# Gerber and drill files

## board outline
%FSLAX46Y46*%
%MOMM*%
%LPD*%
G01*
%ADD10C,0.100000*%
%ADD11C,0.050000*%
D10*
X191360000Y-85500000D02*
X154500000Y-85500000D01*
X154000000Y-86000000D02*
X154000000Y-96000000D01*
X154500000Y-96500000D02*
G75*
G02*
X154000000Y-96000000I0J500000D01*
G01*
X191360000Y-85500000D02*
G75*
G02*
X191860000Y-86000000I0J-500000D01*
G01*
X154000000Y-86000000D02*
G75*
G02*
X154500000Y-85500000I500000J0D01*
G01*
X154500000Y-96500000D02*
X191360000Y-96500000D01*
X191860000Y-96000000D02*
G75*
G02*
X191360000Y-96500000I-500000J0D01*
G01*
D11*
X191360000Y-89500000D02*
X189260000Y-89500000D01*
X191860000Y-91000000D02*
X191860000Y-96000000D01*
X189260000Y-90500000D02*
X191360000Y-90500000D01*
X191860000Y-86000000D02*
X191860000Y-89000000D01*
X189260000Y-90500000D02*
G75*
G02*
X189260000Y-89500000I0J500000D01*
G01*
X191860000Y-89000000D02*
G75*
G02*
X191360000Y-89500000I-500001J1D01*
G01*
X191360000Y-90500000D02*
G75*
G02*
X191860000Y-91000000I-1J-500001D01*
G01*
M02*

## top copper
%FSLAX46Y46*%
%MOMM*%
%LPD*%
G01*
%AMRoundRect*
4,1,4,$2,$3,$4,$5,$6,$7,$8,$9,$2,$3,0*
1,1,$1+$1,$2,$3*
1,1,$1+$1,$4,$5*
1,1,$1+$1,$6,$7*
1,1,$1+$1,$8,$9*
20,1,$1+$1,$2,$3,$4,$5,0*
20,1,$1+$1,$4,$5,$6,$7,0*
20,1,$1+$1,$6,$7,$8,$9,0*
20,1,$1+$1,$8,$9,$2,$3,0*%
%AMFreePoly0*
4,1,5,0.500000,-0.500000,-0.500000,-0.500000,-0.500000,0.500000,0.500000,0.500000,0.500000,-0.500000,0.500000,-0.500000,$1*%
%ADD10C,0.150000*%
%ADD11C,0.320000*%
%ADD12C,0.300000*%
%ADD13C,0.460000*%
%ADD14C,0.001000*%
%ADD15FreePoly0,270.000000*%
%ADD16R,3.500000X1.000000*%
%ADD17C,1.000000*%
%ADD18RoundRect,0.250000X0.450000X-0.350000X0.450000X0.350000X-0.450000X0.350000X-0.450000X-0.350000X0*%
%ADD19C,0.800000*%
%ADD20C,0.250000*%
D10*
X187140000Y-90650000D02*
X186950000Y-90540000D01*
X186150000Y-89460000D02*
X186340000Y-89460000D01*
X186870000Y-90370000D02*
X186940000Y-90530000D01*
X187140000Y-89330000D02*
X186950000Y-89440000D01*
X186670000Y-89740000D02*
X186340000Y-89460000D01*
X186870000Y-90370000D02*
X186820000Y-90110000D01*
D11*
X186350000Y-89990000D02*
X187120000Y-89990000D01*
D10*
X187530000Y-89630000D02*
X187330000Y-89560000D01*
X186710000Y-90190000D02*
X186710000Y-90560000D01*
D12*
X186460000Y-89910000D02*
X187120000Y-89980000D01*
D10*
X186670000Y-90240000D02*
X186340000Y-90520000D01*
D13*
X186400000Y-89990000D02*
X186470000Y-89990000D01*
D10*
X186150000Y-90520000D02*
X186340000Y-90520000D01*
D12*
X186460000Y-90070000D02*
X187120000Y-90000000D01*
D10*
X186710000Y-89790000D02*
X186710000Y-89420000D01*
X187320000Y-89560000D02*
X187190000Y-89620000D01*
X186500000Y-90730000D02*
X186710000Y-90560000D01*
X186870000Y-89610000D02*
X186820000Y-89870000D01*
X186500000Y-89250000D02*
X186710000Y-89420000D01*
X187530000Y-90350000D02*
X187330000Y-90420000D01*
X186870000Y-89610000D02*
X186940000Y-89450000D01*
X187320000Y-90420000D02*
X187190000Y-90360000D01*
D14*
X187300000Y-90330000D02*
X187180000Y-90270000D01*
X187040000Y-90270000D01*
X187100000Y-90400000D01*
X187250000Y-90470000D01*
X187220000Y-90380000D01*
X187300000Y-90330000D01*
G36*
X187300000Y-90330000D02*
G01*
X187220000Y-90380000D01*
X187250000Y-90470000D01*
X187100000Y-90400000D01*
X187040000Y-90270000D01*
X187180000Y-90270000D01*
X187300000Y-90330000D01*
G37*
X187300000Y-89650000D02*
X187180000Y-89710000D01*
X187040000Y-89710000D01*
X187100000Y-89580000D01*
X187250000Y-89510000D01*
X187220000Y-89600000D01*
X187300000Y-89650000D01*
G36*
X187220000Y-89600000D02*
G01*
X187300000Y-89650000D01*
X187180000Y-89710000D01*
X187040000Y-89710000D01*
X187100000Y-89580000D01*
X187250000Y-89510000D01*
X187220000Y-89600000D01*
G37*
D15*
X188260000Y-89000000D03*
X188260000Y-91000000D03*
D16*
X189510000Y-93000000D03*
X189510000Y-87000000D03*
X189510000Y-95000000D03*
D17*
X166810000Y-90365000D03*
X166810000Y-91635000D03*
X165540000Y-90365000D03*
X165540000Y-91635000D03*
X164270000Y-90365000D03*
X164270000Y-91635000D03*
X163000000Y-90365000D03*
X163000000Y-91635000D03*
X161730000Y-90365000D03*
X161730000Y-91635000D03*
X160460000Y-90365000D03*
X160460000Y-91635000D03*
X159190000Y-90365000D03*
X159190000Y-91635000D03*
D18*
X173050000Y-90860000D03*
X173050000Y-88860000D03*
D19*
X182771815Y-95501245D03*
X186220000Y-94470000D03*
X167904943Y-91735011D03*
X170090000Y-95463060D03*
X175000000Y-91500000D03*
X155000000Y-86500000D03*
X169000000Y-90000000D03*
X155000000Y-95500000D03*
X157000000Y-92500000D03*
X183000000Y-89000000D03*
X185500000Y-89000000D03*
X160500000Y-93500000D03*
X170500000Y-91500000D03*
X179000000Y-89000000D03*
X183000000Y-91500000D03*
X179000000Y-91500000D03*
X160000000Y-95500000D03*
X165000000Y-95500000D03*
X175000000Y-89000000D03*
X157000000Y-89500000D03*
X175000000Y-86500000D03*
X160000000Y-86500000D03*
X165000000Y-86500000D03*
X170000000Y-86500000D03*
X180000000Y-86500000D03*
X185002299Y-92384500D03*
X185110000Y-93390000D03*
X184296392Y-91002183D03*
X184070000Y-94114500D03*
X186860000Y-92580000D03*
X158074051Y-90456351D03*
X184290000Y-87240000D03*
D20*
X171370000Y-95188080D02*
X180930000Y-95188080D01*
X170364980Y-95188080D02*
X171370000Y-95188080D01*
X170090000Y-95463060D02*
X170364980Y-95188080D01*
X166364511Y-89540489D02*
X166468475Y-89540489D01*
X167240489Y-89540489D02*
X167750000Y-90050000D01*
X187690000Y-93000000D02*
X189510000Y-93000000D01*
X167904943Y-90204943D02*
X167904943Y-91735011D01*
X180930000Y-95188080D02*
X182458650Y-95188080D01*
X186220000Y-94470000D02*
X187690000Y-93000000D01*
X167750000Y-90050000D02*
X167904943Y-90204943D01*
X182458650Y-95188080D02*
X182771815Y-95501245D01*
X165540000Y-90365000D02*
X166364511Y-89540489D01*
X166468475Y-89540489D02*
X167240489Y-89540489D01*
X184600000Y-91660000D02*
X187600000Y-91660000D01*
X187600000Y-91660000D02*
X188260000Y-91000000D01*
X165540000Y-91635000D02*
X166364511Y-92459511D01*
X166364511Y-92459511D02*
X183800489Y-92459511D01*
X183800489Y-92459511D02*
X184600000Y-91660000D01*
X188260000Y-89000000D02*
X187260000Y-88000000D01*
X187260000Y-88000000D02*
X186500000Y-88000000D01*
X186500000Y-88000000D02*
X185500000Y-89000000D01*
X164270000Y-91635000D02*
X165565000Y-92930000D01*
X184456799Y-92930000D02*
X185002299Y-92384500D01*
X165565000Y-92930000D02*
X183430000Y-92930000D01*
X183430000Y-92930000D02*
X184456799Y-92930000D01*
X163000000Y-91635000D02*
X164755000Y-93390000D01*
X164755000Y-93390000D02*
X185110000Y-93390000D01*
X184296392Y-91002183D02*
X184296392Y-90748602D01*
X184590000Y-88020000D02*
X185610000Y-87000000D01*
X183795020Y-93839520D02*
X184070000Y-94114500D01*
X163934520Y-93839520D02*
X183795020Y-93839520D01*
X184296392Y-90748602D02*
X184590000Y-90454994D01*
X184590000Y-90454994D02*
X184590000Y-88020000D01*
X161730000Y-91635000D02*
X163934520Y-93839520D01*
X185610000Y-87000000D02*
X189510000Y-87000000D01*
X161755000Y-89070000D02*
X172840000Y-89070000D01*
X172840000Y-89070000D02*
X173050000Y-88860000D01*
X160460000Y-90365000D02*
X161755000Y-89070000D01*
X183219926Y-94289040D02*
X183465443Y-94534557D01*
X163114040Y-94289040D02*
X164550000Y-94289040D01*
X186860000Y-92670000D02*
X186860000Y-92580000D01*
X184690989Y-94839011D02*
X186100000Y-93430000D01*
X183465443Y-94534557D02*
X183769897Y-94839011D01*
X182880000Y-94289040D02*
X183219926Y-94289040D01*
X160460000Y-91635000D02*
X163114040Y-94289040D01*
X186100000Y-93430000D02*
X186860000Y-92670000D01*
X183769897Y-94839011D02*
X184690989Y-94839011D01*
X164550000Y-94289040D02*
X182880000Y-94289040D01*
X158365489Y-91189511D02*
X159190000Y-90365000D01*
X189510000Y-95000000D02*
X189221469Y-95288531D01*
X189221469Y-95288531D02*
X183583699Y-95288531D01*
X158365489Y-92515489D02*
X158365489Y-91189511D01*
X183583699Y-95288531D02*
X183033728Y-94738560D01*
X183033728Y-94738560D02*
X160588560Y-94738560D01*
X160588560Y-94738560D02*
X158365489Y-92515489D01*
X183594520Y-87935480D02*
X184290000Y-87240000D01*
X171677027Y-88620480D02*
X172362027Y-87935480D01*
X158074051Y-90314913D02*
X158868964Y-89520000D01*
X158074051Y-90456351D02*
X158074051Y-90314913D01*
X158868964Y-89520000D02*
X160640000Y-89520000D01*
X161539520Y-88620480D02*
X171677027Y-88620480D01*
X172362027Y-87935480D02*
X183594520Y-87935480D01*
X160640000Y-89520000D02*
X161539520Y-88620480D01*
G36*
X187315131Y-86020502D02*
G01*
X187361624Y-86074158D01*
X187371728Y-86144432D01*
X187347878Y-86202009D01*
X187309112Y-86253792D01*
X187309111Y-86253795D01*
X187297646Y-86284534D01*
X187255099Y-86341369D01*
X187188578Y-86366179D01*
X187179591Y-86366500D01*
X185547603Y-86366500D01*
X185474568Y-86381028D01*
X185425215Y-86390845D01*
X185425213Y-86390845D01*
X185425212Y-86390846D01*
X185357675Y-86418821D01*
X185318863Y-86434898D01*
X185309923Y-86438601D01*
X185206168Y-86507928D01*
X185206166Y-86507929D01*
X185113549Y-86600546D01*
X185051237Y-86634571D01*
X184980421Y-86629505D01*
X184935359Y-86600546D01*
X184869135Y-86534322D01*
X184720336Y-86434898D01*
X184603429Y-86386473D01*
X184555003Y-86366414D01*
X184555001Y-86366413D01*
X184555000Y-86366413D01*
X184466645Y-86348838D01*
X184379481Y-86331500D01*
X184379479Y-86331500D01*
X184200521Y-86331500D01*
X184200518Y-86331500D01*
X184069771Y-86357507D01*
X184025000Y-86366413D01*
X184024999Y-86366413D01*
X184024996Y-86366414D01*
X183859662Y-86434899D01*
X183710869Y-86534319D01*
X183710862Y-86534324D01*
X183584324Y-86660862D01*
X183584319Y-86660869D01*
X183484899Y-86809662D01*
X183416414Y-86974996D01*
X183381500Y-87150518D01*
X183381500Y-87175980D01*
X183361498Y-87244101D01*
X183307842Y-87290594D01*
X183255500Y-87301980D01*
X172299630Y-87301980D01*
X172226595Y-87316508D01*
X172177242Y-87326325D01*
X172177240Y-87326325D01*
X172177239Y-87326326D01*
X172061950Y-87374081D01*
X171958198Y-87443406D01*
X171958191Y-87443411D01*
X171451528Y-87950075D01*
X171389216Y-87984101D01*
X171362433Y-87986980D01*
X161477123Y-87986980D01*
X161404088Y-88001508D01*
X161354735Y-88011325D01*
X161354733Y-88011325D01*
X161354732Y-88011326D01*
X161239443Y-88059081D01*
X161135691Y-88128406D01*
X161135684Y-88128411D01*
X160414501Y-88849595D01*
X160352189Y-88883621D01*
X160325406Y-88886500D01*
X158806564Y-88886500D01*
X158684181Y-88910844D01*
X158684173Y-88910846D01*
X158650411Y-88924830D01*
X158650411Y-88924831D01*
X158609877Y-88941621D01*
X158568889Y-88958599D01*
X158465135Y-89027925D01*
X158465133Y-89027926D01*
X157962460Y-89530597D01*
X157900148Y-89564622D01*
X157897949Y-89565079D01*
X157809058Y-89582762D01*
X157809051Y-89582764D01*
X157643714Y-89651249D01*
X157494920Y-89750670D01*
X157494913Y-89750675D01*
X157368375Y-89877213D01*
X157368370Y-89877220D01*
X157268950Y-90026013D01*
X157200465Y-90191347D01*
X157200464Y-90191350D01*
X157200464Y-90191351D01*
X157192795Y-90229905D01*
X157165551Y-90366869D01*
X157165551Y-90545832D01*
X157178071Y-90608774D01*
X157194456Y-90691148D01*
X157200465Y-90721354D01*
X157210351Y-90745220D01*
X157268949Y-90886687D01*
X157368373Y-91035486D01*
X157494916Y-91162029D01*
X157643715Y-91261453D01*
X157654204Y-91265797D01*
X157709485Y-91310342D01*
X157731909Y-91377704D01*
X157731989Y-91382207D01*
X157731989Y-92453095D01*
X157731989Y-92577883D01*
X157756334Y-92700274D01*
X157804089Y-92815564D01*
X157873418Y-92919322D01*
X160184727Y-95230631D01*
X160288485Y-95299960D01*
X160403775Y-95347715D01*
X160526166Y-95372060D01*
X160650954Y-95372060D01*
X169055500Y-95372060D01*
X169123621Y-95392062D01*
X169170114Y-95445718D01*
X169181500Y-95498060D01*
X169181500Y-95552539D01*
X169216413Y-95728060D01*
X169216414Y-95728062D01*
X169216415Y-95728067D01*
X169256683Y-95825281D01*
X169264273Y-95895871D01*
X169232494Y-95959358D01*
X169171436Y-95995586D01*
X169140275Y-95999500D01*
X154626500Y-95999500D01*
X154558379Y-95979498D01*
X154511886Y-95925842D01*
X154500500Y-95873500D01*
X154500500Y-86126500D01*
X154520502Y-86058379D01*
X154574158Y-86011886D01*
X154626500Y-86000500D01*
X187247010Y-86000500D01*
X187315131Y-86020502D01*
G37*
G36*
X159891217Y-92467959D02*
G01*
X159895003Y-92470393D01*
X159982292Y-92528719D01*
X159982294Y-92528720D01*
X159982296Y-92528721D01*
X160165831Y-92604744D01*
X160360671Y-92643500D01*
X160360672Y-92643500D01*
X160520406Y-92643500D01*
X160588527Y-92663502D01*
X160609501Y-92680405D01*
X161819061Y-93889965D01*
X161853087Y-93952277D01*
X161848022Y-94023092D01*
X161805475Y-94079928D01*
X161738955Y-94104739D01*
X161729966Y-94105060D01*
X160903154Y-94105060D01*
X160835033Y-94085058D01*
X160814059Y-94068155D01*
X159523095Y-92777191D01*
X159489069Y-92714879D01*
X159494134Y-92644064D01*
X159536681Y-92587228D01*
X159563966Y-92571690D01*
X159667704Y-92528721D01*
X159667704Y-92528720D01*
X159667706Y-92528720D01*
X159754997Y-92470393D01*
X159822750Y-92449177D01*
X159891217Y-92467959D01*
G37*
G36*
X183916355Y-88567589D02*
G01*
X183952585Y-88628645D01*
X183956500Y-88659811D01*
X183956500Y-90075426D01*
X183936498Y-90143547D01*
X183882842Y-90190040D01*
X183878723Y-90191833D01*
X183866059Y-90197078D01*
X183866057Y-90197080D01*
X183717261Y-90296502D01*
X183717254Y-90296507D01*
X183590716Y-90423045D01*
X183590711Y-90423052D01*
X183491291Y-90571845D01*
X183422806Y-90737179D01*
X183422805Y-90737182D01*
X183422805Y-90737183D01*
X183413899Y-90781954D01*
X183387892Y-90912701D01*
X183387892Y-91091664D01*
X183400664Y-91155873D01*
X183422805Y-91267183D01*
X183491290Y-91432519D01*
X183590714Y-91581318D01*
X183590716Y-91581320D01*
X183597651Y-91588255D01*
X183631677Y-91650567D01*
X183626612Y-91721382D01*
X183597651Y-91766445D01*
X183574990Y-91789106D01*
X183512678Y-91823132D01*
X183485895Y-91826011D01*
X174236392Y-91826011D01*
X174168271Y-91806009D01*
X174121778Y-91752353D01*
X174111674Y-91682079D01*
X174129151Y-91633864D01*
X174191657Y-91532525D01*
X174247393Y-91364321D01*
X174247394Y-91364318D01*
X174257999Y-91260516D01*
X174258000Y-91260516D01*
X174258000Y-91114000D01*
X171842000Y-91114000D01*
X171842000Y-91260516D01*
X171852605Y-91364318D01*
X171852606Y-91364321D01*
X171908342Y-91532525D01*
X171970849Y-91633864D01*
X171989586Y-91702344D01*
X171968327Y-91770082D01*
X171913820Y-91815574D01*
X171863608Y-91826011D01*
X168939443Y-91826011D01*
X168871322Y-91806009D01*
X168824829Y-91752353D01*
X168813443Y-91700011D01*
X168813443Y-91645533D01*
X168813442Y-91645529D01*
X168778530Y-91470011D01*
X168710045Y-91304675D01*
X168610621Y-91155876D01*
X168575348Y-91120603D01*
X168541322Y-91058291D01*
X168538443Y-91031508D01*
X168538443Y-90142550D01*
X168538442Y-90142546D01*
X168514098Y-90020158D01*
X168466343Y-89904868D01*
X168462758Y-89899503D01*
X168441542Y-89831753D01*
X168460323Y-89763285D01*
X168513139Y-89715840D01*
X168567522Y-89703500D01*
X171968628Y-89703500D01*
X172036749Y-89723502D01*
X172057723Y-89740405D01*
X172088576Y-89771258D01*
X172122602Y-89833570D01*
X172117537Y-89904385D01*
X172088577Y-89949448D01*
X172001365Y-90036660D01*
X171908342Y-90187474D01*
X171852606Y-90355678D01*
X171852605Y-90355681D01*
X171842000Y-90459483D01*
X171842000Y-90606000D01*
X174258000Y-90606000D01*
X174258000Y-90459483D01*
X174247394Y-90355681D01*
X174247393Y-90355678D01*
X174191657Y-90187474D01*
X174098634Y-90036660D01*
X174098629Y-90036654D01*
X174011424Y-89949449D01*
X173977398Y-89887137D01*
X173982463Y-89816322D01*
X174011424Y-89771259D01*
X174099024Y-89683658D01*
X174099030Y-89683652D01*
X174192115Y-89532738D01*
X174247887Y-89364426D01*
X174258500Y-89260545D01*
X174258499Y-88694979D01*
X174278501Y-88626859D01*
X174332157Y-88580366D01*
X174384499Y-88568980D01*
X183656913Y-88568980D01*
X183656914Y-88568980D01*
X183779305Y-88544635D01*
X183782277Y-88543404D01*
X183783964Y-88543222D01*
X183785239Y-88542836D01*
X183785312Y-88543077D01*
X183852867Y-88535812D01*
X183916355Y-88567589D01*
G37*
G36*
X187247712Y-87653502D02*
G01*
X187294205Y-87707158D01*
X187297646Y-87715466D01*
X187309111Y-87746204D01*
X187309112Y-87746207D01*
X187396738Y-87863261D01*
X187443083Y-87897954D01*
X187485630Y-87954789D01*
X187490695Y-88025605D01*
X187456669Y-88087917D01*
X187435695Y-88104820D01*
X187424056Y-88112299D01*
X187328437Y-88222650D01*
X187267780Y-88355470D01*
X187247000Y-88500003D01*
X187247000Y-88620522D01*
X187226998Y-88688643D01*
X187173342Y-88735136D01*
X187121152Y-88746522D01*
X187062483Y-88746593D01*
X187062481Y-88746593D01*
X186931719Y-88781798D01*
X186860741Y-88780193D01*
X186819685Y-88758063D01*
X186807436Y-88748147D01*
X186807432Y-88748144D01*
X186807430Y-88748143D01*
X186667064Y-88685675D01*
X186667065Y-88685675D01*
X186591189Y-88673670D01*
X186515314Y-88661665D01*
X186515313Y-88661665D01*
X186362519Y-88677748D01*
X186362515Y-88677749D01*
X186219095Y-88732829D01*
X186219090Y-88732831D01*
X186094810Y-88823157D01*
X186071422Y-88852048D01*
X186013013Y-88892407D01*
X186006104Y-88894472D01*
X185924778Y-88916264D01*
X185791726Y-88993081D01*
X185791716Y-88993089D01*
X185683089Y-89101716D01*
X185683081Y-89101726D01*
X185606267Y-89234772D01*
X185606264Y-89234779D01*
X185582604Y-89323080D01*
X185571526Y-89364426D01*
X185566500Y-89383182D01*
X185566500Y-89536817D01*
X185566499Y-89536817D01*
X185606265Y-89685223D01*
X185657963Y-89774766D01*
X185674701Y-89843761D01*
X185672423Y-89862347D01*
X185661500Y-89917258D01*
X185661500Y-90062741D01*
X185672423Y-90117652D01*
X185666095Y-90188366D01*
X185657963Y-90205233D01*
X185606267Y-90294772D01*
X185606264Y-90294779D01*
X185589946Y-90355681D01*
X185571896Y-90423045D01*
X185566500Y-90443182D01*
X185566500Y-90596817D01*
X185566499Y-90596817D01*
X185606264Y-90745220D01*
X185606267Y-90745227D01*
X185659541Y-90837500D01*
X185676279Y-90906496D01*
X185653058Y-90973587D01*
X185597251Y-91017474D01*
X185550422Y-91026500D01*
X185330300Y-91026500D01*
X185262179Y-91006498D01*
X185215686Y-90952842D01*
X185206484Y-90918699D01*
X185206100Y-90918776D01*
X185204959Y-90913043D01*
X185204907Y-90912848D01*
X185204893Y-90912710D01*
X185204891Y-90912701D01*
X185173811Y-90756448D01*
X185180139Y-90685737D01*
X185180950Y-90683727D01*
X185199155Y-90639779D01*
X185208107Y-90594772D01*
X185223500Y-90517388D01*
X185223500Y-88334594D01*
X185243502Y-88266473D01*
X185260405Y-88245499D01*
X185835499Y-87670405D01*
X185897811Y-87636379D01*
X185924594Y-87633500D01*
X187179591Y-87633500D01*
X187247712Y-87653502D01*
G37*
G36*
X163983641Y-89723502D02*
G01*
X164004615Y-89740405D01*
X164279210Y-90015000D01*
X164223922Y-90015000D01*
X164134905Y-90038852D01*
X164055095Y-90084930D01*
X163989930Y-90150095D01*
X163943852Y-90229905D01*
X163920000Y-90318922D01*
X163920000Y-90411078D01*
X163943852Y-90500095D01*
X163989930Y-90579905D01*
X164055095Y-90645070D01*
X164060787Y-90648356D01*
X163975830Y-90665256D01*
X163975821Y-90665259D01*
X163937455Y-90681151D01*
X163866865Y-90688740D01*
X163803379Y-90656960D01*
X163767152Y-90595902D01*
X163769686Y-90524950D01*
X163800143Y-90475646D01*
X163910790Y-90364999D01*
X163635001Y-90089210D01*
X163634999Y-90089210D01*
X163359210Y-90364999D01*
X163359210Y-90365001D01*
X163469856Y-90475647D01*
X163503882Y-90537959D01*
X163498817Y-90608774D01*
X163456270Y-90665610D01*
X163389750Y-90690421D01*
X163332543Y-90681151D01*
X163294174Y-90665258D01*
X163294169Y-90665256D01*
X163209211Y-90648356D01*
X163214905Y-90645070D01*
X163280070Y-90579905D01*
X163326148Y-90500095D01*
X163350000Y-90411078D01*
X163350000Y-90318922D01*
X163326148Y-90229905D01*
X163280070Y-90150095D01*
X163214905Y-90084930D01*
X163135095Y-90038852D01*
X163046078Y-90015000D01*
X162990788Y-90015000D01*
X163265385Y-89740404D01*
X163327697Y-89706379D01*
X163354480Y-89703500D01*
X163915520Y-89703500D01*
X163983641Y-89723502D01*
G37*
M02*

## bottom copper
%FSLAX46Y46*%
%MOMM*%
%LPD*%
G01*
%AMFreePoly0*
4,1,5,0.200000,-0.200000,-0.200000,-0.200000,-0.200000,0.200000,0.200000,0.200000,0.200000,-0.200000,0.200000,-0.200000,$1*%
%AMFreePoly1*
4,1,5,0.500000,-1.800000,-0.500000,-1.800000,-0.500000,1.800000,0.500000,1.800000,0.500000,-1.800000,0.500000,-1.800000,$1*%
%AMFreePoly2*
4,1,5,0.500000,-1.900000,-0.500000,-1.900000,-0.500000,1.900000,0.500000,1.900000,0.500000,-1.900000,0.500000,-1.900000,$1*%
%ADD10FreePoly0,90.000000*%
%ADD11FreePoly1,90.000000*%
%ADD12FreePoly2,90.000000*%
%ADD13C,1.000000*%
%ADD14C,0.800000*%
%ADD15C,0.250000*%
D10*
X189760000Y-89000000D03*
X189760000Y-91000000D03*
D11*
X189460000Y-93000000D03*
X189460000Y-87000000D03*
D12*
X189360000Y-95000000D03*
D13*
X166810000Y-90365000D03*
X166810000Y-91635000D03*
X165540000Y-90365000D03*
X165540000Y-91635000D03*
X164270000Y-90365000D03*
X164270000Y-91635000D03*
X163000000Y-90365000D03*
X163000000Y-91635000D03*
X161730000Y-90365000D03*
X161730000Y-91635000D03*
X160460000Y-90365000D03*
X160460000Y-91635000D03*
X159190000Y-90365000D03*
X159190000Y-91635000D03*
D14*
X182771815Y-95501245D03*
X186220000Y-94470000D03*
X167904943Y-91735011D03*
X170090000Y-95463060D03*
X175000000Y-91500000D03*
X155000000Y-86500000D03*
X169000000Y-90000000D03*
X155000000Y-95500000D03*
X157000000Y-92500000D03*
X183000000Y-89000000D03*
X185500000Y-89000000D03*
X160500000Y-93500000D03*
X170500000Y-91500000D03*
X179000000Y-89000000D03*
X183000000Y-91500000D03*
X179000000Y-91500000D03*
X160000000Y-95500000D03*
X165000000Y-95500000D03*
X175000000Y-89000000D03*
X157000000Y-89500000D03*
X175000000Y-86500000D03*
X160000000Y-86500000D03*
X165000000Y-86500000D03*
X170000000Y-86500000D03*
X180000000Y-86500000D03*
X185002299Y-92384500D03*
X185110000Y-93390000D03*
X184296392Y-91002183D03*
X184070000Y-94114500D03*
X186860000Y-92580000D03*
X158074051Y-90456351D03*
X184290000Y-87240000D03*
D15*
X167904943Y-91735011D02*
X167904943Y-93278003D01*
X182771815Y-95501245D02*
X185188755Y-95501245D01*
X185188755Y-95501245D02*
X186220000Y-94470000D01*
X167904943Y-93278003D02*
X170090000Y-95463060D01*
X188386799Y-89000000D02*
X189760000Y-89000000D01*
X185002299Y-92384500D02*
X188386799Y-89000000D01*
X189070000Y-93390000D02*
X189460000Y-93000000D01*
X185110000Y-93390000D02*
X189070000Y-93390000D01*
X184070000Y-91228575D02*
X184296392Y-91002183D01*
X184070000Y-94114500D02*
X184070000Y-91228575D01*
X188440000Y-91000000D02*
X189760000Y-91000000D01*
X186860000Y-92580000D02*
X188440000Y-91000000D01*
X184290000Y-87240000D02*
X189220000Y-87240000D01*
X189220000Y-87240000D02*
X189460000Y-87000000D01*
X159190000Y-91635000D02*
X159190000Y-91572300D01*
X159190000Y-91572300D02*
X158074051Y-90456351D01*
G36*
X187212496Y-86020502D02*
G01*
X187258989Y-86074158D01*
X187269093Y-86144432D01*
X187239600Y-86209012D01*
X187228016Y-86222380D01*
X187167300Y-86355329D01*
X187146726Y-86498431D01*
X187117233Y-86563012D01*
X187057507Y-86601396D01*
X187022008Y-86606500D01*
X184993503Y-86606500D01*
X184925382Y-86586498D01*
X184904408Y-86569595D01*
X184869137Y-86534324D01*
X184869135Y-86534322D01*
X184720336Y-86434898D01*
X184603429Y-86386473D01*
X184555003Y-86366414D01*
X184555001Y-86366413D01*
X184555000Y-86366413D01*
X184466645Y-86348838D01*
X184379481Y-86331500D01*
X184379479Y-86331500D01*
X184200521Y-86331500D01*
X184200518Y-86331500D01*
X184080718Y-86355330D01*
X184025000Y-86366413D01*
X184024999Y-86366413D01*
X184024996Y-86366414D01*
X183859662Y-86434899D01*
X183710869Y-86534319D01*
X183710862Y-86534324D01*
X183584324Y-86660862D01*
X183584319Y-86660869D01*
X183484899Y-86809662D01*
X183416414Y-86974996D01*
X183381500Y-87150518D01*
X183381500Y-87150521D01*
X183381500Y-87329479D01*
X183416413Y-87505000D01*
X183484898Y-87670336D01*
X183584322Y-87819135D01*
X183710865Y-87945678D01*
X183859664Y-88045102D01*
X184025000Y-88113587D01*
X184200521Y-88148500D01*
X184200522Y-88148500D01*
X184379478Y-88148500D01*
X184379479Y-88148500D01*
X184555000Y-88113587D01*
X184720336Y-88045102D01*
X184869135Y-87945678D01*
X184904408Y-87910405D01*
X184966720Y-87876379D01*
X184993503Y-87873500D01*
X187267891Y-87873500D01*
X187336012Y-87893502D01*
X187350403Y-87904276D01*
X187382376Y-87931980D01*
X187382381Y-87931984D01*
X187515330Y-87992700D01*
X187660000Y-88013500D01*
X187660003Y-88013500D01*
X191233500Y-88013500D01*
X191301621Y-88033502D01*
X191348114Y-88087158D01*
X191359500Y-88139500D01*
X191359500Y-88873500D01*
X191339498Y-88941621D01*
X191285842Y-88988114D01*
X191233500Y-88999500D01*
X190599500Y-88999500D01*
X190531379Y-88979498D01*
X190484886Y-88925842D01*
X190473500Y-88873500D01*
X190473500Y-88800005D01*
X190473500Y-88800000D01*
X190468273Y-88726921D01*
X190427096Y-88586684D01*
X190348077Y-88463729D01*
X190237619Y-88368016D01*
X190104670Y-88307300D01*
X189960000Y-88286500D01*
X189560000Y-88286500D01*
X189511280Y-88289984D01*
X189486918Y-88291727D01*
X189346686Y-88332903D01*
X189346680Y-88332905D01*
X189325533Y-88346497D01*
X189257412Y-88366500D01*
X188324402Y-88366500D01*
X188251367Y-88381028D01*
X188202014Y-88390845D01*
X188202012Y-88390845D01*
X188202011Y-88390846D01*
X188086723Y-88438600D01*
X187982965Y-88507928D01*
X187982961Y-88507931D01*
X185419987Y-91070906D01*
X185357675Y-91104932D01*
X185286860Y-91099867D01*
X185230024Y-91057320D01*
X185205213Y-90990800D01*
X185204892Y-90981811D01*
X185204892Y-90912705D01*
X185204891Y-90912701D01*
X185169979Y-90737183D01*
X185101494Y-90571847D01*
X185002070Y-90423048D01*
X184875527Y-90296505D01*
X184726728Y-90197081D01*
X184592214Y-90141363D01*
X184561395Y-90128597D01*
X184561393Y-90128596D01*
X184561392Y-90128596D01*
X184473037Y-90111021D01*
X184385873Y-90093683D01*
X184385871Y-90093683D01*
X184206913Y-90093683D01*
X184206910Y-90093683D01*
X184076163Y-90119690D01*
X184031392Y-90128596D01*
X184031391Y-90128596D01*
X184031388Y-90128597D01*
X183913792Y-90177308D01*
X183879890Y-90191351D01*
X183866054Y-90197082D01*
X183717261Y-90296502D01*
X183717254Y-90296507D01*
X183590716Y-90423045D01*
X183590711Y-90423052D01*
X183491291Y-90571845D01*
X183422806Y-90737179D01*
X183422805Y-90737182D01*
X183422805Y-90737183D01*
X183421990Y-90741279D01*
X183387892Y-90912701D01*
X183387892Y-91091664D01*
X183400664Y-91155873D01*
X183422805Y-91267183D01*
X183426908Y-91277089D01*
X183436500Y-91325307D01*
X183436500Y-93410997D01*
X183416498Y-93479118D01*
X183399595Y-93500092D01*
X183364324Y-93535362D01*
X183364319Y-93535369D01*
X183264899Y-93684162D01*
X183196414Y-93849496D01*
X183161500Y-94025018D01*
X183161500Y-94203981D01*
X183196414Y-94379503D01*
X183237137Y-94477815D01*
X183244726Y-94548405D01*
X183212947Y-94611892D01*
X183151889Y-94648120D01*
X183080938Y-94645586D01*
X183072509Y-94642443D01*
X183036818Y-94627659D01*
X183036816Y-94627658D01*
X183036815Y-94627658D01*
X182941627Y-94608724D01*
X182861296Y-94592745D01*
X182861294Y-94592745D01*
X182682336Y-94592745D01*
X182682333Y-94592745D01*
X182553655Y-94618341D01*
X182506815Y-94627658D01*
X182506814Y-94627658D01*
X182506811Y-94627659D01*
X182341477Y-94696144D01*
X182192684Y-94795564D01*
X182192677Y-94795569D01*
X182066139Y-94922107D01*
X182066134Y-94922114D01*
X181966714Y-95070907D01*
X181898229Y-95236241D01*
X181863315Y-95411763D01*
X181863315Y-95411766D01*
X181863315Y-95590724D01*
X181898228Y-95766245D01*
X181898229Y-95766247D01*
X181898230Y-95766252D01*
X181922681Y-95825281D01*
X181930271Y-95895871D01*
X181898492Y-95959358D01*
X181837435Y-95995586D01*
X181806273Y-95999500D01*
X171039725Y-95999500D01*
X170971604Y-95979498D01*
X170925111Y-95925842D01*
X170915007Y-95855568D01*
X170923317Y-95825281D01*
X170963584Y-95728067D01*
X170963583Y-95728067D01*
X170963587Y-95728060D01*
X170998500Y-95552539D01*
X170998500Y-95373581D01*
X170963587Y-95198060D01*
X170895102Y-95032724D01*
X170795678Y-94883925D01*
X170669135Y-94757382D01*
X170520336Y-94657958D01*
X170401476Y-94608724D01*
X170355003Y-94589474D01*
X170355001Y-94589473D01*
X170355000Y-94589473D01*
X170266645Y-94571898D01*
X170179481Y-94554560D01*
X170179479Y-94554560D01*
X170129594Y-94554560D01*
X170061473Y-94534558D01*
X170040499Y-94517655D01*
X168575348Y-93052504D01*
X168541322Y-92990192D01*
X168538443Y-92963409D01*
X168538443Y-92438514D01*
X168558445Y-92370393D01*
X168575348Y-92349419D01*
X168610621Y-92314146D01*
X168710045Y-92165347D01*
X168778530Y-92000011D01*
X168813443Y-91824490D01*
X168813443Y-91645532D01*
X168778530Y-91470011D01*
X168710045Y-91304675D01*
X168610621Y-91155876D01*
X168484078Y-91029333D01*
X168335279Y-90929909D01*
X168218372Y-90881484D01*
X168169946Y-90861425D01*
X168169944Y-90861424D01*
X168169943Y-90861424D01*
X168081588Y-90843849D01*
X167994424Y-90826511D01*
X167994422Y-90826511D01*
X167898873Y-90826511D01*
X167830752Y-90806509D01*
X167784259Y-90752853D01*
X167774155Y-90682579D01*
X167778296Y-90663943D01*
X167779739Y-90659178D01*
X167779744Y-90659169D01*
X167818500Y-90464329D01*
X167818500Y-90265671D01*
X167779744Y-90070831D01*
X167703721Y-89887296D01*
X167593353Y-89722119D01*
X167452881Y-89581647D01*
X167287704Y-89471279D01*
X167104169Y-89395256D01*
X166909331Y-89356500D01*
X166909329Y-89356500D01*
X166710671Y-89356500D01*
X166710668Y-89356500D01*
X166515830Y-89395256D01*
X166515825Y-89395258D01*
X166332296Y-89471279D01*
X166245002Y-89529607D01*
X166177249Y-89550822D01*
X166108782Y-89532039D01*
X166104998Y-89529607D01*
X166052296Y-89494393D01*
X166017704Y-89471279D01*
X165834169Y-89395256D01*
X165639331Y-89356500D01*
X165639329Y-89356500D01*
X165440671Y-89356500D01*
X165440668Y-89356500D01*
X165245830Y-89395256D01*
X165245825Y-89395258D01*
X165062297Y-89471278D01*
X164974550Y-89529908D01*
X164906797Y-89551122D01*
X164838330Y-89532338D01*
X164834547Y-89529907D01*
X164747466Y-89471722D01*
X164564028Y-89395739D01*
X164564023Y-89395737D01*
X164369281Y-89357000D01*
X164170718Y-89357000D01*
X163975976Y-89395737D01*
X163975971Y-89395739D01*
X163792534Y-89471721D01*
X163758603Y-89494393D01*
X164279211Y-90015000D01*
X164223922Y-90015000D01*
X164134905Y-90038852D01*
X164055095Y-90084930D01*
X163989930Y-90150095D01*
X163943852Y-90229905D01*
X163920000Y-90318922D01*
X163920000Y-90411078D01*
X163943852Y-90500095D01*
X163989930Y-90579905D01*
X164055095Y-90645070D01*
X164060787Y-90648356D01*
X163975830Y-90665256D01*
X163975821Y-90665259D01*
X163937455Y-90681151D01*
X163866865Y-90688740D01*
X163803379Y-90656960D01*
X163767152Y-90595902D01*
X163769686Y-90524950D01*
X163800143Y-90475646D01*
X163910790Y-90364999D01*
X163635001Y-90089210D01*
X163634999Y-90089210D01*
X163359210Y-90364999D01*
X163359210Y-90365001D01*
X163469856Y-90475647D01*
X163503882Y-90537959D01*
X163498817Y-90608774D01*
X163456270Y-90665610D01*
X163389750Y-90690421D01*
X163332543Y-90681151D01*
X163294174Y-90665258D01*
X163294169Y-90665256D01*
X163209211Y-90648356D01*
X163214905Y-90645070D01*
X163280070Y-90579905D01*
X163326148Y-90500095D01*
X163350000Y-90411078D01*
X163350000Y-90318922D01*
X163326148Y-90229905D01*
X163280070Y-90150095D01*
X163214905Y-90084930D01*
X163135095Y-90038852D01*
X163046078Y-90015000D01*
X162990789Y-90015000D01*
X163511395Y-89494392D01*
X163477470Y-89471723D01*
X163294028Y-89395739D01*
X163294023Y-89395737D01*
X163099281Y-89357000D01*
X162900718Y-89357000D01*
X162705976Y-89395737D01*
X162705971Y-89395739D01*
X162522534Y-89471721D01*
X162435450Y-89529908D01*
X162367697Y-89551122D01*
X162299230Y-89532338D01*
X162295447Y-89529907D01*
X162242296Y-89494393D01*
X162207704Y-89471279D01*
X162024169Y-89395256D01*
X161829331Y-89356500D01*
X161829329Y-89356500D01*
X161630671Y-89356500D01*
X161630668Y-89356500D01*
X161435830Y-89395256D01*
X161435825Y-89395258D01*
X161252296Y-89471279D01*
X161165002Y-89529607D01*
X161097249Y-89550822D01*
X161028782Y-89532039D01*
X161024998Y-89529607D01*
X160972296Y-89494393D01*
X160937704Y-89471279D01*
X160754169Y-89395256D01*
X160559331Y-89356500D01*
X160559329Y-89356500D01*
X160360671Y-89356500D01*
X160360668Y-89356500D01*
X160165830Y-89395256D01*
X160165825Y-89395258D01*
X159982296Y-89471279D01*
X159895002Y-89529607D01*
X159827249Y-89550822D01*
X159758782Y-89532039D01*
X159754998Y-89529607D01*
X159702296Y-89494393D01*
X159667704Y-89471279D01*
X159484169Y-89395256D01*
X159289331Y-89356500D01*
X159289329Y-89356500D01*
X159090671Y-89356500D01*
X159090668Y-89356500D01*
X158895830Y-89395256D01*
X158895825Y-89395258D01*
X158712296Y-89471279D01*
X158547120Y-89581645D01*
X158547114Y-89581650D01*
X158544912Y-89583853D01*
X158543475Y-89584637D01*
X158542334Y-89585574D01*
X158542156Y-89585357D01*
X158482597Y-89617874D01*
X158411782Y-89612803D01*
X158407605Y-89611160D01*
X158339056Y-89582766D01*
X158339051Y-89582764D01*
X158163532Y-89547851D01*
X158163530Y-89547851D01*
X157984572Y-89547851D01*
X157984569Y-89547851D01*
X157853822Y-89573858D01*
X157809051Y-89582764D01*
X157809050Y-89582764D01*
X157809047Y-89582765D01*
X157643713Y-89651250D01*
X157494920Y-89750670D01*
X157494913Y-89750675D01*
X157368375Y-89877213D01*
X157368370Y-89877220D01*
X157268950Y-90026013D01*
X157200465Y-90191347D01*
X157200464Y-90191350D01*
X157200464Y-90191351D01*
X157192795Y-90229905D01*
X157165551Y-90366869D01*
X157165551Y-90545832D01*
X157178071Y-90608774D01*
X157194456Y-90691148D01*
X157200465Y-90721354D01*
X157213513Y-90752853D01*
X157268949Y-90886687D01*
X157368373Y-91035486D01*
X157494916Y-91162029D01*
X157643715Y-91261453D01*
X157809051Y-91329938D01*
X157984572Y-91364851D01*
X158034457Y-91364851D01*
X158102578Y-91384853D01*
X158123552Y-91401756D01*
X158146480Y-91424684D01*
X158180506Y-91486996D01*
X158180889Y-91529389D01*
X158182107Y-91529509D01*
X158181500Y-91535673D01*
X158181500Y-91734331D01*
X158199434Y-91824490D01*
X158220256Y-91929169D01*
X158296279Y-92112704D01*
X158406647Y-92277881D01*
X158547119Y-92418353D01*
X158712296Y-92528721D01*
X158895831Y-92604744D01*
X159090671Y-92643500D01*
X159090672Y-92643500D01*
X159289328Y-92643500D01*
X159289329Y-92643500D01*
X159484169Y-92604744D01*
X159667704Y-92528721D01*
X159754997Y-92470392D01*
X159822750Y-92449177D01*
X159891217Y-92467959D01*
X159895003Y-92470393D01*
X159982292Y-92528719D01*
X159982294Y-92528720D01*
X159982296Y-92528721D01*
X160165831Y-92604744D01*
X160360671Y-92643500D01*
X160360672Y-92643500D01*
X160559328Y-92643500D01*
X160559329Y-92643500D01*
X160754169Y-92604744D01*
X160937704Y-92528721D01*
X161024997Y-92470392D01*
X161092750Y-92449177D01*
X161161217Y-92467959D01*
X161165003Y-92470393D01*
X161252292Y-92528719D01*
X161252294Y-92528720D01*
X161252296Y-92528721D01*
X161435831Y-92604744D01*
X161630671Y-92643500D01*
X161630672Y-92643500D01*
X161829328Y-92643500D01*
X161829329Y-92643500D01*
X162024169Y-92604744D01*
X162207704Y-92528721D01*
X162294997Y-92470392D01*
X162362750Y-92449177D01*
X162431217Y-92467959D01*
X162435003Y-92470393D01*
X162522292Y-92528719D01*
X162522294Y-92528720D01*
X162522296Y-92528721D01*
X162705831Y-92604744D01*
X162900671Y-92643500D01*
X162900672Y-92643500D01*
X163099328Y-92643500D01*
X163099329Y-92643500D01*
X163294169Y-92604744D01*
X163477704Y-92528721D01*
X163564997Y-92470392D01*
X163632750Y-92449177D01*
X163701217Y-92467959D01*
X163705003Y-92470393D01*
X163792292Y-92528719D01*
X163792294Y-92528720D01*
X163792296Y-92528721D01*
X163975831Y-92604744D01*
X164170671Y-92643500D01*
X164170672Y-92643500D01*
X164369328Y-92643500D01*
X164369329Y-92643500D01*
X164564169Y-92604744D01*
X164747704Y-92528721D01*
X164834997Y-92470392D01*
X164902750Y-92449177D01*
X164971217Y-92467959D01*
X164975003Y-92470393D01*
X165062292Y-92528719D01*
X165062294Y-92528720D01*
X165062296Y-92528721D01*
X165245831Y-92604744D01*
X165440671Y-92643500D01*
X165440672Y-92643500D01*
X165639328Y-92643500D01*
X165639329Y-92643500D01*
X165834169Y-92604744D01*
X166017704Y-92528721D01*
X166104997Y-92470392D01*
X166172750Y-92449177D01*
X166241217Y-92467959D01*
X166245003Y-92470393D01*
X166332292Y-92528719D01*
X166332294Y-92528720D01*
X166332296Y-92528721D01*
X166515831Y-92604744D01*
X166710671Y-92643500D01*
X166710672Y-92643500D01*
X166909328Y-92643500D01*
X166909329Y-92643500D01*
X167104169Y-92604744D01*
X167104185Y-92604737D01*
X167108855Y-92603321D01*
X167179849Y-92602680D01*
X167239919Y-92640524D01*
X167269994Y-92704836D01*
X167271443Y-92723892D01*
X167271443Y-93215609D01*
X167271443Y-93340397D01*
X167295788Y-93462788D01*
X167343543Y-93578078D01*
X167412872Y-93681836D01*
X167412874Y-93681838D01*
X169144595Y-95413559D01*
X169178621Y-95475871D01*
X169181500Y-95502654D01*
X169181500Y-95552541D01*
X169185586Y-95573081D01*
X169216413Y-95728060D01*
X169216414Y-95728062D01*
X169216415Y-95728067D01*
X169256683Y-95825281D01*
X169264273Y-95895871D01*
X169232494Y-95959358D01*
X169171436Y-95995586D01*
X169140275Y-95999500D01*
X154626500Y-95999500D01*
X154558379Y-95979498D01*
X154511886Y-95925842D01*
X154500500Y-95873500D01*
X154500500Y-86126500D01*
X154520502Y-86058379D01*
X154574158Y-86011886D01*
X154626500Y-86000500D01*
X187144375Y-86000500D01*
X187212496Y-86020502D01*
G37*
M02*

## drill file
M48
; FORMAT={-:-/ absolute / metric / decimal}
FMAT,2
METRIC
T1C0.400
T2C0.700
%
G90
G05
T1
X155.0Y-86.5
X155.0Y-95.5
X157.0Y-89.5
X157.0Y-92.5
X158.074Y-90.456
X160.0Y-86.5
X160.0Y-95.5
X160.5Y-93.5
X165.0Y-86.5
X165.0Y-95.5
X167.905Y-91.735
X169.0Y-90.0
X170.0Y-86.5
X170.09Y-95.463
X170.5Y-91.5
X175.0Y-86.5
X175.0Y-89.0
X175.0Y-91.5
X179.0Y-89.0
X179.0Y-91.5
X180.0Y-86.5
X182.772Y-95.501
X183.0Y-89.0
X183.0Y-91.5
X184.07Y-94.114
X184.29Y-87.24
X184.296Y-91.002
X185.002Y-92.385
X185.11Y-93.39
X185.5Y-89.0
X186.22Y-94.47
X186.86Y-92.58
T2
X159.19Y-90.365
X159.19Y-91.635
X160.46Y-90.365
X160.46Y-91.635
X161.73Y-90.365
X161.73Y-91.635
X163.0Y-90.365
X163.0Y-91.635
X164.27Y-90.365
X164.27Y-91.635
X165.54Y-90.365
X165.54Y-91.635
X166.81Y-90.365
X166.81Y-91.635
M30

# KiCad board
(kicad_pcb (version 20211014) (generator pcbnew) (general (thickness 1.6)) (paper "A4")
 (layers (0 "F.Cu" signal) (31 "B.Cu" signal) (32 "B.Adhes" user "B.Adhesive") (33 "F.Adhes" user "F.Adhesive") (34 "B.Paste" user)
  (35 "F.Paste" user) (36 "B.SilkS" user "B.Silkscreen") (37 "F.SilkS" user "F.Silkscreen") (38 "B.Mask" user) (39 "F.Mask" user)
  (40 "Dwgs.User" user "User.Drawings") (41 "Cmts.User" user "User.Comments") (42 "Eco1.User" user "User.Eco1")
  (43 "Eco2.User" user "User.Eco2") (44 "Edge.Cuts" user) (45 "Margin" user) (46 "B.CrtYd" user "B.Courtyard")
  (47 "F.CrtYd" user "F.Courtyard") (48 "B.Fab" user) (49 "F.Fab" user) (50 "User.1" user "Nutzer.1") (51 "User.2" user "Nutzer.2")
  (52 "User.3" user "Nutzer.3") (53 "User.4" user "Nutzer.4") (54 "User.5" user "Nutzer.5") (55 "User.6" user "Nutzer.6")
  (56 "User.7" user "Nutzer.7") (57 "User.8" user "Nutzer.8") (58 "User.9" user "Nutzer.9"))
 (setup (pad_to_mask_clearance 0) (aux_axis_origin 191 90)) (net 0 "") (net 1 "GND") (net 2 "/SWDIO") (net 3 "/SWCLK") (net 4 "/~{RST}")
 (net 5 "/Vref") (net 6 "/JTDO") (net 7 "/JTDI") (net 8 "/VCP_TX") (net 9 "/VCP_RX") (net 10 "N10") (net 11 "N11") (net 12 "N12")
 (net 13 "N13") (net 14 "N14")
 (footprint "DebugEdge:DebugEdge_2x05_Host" (layer "F.Cu") (at 191.86 91 -90)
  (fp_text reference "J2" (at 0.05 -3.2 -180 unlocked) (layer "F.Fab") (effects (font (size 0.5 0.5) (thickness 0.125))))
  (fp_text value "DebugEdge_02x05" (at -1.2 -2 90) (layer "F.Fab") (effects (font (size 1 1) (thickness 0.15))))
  (fp_line (start -0.35 4.72) (end -0.46 4.91) (layer "F.Cu") (width 0.15))
  (fp_line (start -1.54 5.71) (end -1.54 5.52) (layer "F.Cu") (width 0.15))
  (fp_line (start -0.63 4.99) (end -0.47 4.92) (layer "F.Cu") (width 0.15))
  (fp_line (start -1.67 4.72) (end -1.56 4.91) (layer "F.Cu") (width 0.15))
  (fp_line (start -1.26 5.19) (end -1.54 5.52) (layer "F.Cu") (width 0.15))
  (fp_line (start -0.63 4.99) (end -0.89 5.04) (layer "F.Cu") (width 0.15))
  (fp_line (start -1.01 5.51) (end -1.01 4.74) (layer "F.Cu") (width 0.32))
  (fp_line (start -1.37 4.33) (end -1.44 4.53) (layer "F.Cu") (width 0.15))
  (fp_line (start -0.81 5.15) (end -0.44 5.15) (layer "F.Cu") (width 0.15))
  (fp_line (start -1.09 5.4) (end -1.02 4.74) (layer "F.Cu") (width 0.3))
  (fp_line (start -0.76 5.19) (end -0.48 5.52) (layer "F.Cu") (width 0.15))
  (fp_line (start -1.01 5.46) (end -1.01 5.39) (layer "F.Cu") (width 0.46))
  (fp_line (start -0.48 5.71) (end -0.48 5.52) (layer "F.Cu") (width 0.15))
  (fp_line (start -0.93 5.4) (end -1 4.74) (layer "F.Cu") (width 0.3))
  (fp_line (start -1.21 5.15) (end -1.58 5.15) (layer "F.Cu") (width 0.15))
  (fp_line (start -1.44 4.54) (end -1.38 4.67) (layer "F.Cu") (width 0.15))
  (fp_line (start -0.27 5.36) (end -0.44 5.15) (layer "F.Cu") (width 0.15))
  (fp_line (start -1.39 4.99) (end -1.13 5.04) (layer "F.Cu") (width 0.15))
  (fp_line (start -1.75 5.36) (end -1.58 5.15) (layer "F.Cu") (width 0.15))
  (fp_line (start -0.65 4.33) (end -0.58 4.53) (layer "F.Cu") (width 0.15))
  (fp_line (start -1.39 4.99) (end -1.55 4.92) (layer "F.Cu") (width 0.15))
  (fp_line (start -0.58 4.54) (end -0.64 4.67) (layer "F.Cu") (width 0.15))
  (fp_poly
   (pts (xy -0.67 4.56) (xy -0.73 4.68) (xy -0.73 4.82) (xy -0.6 4.76) (xy -0.53 4.61) (xy -0.62 4.64)) (layer "F.Cu") (width 0.001)
   (fill solid))
  (fp_poly
   (pts (xy -1.35 4.56) (xy -1.29 4.68) (xy -1.29 4.82) (xy -1.42 4.76) (xy -1.49 4.61) (xy -1.4 4.64)) (layer "F.Cu") (width 0.001)
   (fill solid))
  (fp_line (start -1.5 0.5) (end -1.5 2.6) (layer "Edge.Cuts") (width 0.05))
  (fp_line (start 0 0) (end 5 0) (layer "Edge.Cuts") (width 0.05))
  (fp_line (start -0.5 2.6) (end -0.5 0.5) (layer "Edge.Cuts") (width 0.05))
  (fp_line (start -5 0) (end -2 0) (layer "Edge.Cuts") (width 0.05))
  (fp_arc (start -0.5 2.6) (mid -1 3.1) (end -1.5 2.6) (layer "Edge.Cuts") (width 0.05))
  (fp_arc (start -2 0) (mid -1.646447 0.146447) (end -1.5 0.5) (layer "Edge.Cuts") (width 0.05))
  (fp_arc (start -0.5 0.5) (mid -0.353553 0.146447) (end 0 0) (layer "Edge.Cuts") (width 0.05))
  (pad "1" smd custom locked (at -2 3.6 270) (size 1 1) (layers "F.Cu" "F.Mask") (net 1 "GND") (zone_connect 0)
   (options (clearance outline) (anchor rect)) (primitives))
  (pad "2" smd custom locked (at 0 3.6 270) (size 1 1) (layers "F.Cu" "F.Mask") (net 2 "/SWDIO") (zone_connect 0)
   (options (clearance outline) (anchor rect)) (primitives))
  (pad "3" smd custom locked (at -2 2.1 90) (size 0.4 0.4) (layers "B.Cu" "B.Mask") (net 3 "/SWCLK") (zone_connect 0)
   (options (clearance outline) (anchor rect)) (primitives))
  (pad "4" smd custom locked (at 0 2.1 90) (size 0.4 0.4) (layers "B.Cu" "B.Mask") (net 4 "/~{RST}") (zone_connect 0)
   (options (clearance outline) (anchor rect)) (primitives))
  (pad "5" smd rect locked (at 2 2.35 270) (size 1 3.5) (layers "F.Cu" "F.Mask") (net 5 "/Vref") (zone_connect 0))
  (pad "6" smd custom locked (at 2 2.4 90) (size 1 3.6) (layers "B.Cu" "B.Mask") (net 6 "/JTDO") (zone_connect 0)
   (options (clearance outline) (anchor rect)) (primitives))
  (pad "7" smd rect locked (at -4 2.35 270) (size 1 3.5) (layers "F.Cu" "F.Mask") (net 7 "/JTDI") (zone_connect 0))
  (pad "8" smd custom locked (at -4 2.4 90) (size 1 3.6) (layers "B.Cu" "B.Mask") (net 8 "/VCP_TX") (zone_connect 0)
   (options (clearance outline) (anchor rect)) (primitives))
  (pad "9" smd rect locked (at 4 2.35 270) (size 1 3.5) (layers "F.Cu" "F.Mask") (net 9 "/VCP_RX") (zone_connect 0))
  (pad "10" smd custom locked (at 4 2.5 90) (size 1 3.8) (layers "B.Cu" "B.Mask") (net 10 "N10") (zone_connect 0)
   (options (clearance outline) (anchor rect)) (primitives)))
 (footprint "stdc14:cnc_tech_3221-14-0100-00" (layer "F.Cu") (at 163 91)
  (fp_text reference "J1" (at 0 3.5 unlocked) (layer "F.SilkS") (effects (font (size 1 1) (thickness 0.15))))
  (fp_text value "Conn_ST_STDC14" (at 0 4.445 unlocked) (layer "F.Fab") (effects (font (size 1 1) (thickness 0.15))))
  (pad "1" thru_hole circle (at 3.81 -0.635) (size 1 1) (drill 0.7) (layers *.Cu *.Mask) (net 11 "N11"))
  (pad "2" thru_hole circle (at 3.81 0.635) (size 1 1) (drill 0.7) (layers *.Cu *.Mask) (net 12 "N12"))
  (pad "3" thru_hole circle (at 2.54 -0.635) (size 1 1) (drill 0.7) (layers *.Cu *.Mask) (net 5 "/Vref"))
  (pad "4" thru_hole circle (at 2.54 0.635) (size 1 1) (drill 0.7) (layers *.Cu *.Mask) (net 2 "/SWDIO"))
  (pad "5" thru_hole circle (at 1.27 -0.635) (size 1 1) (drill 0.7) (layers *.Cu *.Mask) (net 1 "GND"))
  (pad "6" thru_hole circle (at 1.27 0.635) (size 1 1) (drill 0.7) (layers *.Cu *.Mask) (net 3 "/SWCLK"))
  (pad "7" thru_hole circle (at 0 -0.635) (size 1 1) (drill 0.7) (layers *.Cu *.Mask) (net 1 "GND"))
  (pad "8" thru_hole circle (at 0 0.635) (size 1 1) (drill 0.7) (layers *.Cu *.Mask) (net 6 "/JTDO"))
  (pad "9" thru_hole circle (at -1.27 -0.635) (size 1 1) (drill 0.7) (layers *.Cu *.Mask) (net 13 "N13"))
  (pad "10" thru_hole circle (at -1.27 0.635) (size 1 1) (drill 0.7) (layers *.Cu *.Mask) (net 7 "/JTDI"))
  (pad "11" thru_hole circle (at -2.54 -0.635) (size 1 1) (drill 0.7) (layers *.Cu *.Mask) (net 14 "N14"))
  (pad "12" thru_hole circle (at -2.54 0.635) (size 1 1) (drill 0.7) (layers *.Cu *.Mask) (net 4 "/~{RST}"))
  (pad "13" thru_hole circle (at -3.81 -0.635) (size 1 1) (drill 0.7) (layers *.Cu *.Mask) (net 9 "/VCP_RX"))
  (pad "14" thru_hole circle (at -3.81 0.635) (size 1 1) (drill 0.7) (layers *.Cu *.Mask) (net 8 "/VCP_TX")))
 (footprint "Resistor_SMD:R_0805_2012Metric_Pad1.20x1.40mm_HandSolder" (layer "F.Cu") (at 173.05 89.86 90)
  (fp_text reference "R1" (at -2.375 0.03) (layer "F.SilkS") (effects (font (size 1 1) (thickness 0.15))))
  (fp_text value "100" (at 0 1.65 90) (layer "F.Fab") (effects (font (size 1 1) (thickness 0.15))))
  (pad "1" smd roundrect (at -1 0 90) (size 1.2 1.4) (layers "F.Cu" "F.Paste" "F.Mask") (roundrect_rratio 0.208333) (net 1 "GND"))
  (pad "2" smd roundrect (at 1 0 90) (size 1.2 1.4) (layers "F.Cu" "F.Paste" "F.Mask") (roundrect_rratio 0.208333) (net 14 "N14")))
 (gr_line (start 191.36 85.5) (end 154.5 85.5) (layer "Edge.Cuts") (width 0.1))
 (gr_line (start 154 86) (end 154 96) (layer "Edge.Cuts") (width 0.1))
 (gr_arc (start 154.5 96.5) (mid 154.146447 96.353553) (end 154 96) (layer "Edge.Cuts") (width 0.1))
 (gr_arc (start 191.36 85.5) (mid 191.713553 85.646447) (end 191.86 86) (layer "Edge.Cuts") (width 0.1))
 (gr_arc (start 154 86) (mid 154.146447 85.646447) (end 154.5 85.5) (layer "Edge.Cuts") (width 0.1))
 (gr_line (start 154.5 96.5) (end 191.36 96.5) (layer "Edge.Cuts") (width 0.1))
 (gr_arc (start 191.86 96) (mid 191.713553 96.353553) (end 191.36 96.5) (layer "Edge.Cuts") (width 0.1))
 (segment (start 171.37 95.18808) (end 180.93 95.18808) (width 0.25) (layer "F.Cu") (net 5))
 (segment (start 170.36498 95.18808) (end 171.37 95.18808) (width 0.25) (layer "F.Cu") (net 5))
 (segment (start 170.09 95.46306) (end 170.36498 95.18808) (width 0.25) (layer "F.Cu") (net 5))
 (segment (start 166.364511 89.540489) (end 166.468475 89.540489) (width 0.25) (layer "F.Cu") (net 5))
 (segment (start 167.240489 89.540489) (end 167.75 90.05) (width 0.25) (layer "F.Cu") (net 5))
 (segment (start 187.69 93) (end 189.51 93) (width 0.25) (layer "F.Cu") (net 5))
 (segment (start 167.904943 90.204943) (end 167.904943 91.735011) (width 0.25) (layer "F.Cu") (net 5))
 (segment (start 180.93 95.18808) (end 182.45865 95.18808) (width 0.25) (layer "F.Cu") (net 5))
 (segment (start 186.22 94.47) (end 187.69 93) (width 0.25) (layer "F.Cu") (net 5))
 (segment (start 167.75 90.05) (end 167.904943 90.204943) (width 0.25) (layer "F.Cu") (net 5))
 (segment (start 182.45865 95.18808) (end 182.771815 95.501245) (width 0.25) (layer "F.Cu") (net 5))
 (segment (start 165.54 90.365) (end 166.364511 89.540489) (width 0.25) (layer "F.Cu") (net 5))
 (segment (start 166.468475 89.540489) (end 167.240489 89.540489) (width 0.25) (layer "F.Cu") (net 5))
 (via (at 182.771815 95.501245) (size 0.8) (drill 0.4) (layers "F.Cu" "B.Cu") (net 5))
 (via (at 186.22 94.47) (size 0.8) (drill 0.4) (layers "F.Cu" "B.Cu") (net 5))
 (via (at 167.904943 91.735011) (size 0.8) (drill 0.4) (layers "F.Cu" "B.Cu") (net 5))
 (via (at 170.09 95.46306) (size 0.8) (drill 0.4) (layers "F.Cu" "B.Cu") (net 5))
 (segment (start 167.904943 91.735011) (end 167.904943 93.278003) (width 0.25) (layer "B.Cu") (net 5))
 (segment (start 182.771815 95.501245) (end 185.188755 95.501245) (width 0.25) (layer "B.Cu") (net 5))
 (segment (start 185.188755 95.501245) (end 186.22 94.47) (width 0.25) (layer "B.Cu") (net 5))
 (segment (start 167.904943 93.278003) (end 170.09 95.46306) (width 0.25) (layer "B.Cu") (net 5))
 (segment (start 184.6 91.66) (end 187.6 91.66) (width 0.25) (layer "F.Cu") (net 2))
 (segment (start 187.6 91.66) (end 188.26 91) (width 0.25) (layer "F.Cu") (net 2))
 (segment (start 165.54 91.635) (end 166.364511 92.459511) (width 0.25) (layer "F.Cu") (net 2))
 (segment (start 166.364511 92.459511) (end 183.800489 92.459511) (width 0.25) (layer "F.Cu") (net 2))
 (segment (start 183.800489 92.459511) (end 184.6 91.66) (width 0.25) (layer "F.Cu") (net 2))
 (segment (start 188.26 89) (end 187.26 88) (width 0.25) (layer "F.Cu") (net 1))
 (segment (start 187.26 88) (end 186.5 88) (width 0.25) (layer "F.Cu") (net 1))
 (segment (start 186.5 88) (end 185.5 89) (width 0.25) (layer "F.Cu") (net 1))
 (via (at 175 91.5) (size 0.8) (drill 0.4) (layers "F.Cu" "B.Cu") (free) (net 1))
 (via (at 155 86.5) (size 0.8) (drill 0.4) (layers "F.Cu" "B.Cu") (free) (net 1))
 (via (at 169 90) (size 0.8) (drill 0.4) (layers "F.Cu" "B.Cu") (free) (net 1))
 (via (at 155 95.5) (size 0.8) (drill 0.4) (layers "F.Cu" "B.Cu") (free) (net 1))
 (via (at 157 92.5) (size 0.8) (drill 0.4) (layers "F.Cu" "B.Cu") (free) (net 1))
 (via (at 183 89) (size 0.8) (drill 0.4) (layers "F.Cu" "B.Cu") (free) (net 1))
 (via (at 185.5 89) (size 0.8) (drill 0.4) (layers "F.Cu" "B.Cu") (free) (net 1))
 (via (at 160.5 93.5) (size 0.8) (drill 0.4) (layers "F.Cu" "B.Cu") (free) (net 1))
 (via (at 170.5 91.5) (size 0.8) (drill 0.4) (layers "F.Cu" "B.Cu") (free) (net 1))
 (via (at 179 89) (size 0.8) (drill 0.4) (layers "F.Cu" "B.Cu") (free) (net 1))
 (via (at 183 91.5) (size 0.8) (drill 0.4) (layers "F.Cu" "B.Cu") (free) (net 1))
 (via (at 179 91.5) (size 0.8) (drill 0.4) (layers "F.Cu" "B.Cu") (free) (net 1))
 (via (at 160 95.5) (size 0.8) (drill 0.4) (layers "F.Cu" "B.Cu") (free) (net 1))
 (via (at 165 95.5) (size 0.8) (drill 0.4) (layers "F.Cu" "B.Cu") (free) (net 1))
 (via (at 175 89) (size 0.8) (drill 0.4) (layers "F.Cu" "B.Cu") (free) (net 1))
 (via (at 157 89.5) (size 0.8) (drill 0.4) (layers "F.Cu" "B.Cu") (free) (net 1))
 (via (at 175 86.5) (size 0.8) (drill 0.4) (layers "F.Cu" "B.Cu") (free) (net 1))
 (via (at 160 86.5) (size 0.8) (drill 0.4) (layers "F.Cu" "B.Cu") (free) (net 1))
 (via (at 165 86.5) (size 0.8) (drill 0.4) (layers "F.Cu" "B.Cu") (free) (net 1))
 (via (at 170 86.5) (size 0.8) (drill 0.4) (layers "F.Cu" "B.Cu") (free) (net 1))
 (via (at 180 86.5) (size 0.8) (drill 0.4) (layers "F.Cu" "B.Cu") (free) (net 1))
 (segment (start 164.27 91.635) (end 165.565 92.93) (width 0.25) (layer "F.Cu") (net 3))
 (segment (start 184.456799 92.93) (end 185.002299 92.3845) (width 0.25) (layer "F.Cu") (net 3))
 (segment (start 165.565 92.93) (end 183.43 92.93) (width 0.25) (layer "F.Cu") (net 3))
 (segment (start 183.43 92.93) (end 184.456799 92.93) (width 0.25) (layer "F.Cu") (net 3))
 (via (at 185.002299 92.3845) (size 0.8) (drill 0.4) (layers "F.Cu" "B.Cu") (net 3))
 (segment (start 188.386799 89) (end 189.76 89) (width 0.25) (layer "B.Cu") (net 3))
 (segment (start 185.002299 92.3845) (end 188.386799 89) (width 0.25) (layer "B.Cu") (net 3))
 (segment (start 163 91.635) (end 164.755 93.39) (width 0.25) (layer "F.Cu") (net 6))
 (segment (start 164.755 93.39) (end 185.11 93.39) (width 0.25) (layer "F.Cu") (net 6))
 (via (at 185.11 93.39) (size 0.8) (drill 0.4) (layers "F.Cu" "B.Cu") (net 6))
 (segment (start 189.07 93.39) (end 189.46 93) (width 0.25) (layer "B.Cu") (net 6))
 (segment (start 185.11 93.39) (end 189.07 93.39) (width 0.25) (layer "B.Cu") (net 6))
 (segment (start 184.296392 91.002183) (end 184.296392 90.748602) (width 0.25) (layer "F.Cu") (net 7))
 (segment (start 184.59 88.02) (end 185.61 87) (width 0.25) (layer "F.Cu") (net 7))
 (segment (start 183.79502 93.83952) (end 184.07 94.1145) (width 0.25) (layer "F.Cu") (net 7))
 (segment (start 163.93452 93.83952) (end 183.79502 93.83952) (width 0.25) (layer "F.Cu") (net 7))
 (segment (start 184.296392 90.748602) (end 184.59 90.454994) (width 0.25) (layer "F.Cu") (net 7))
 (segment (start 184.59 90.454994) (end 184.59 88.02) (width 0.25) (layer "F.Cu") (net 7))
 (segment (start 161.73 91.635) (end 163.93452 93.83952) (width 0.25) (layer "F.Cu") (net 7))
 (segment (start 185.61 87) (end 189.51 87) (width 0.25) (layer "F.Cu") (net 7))
 (via (at 184.296392 91.002183) (size 0.8) (drill 0.4) (layers "F.Cu" "B.Cu") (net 7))
 (via (at 184.07 94.1145) (size 0.8) (drill 0.4) (layers "F.Cu" "B.Cu") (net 7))
 (segment (start 184.07 91.228575) (end 184.296392 91.002183) (width 0.25) (layer "B.Cu") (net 7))
 (segment (start 184.07 94.1145) (end 184.07 91.228575) (width 0.25) (layer "B.Cu") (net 7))
 (segment (start 161.755 89.07) (end 172.84 89.07) (width 0.25) (layer "F.Cu") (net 14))
 (segment (start 172.84 89.07) (end 173.05 88.86) (width 0.25) (layer "F.Cu") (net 14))
 (segment (start 160.46 90.365) (end 161.755 89.07) (width 0.25) (layer "F.Cu") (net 14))
 (segment (start 183.219926 94.28904) (end 183.465443 94.534557) (width 0.25) (layer "F.Cu") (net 4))
 (segment (start 163.11404 94.28904) (end 164.55 94.28904) (width 0.25) (layer "F.Cu") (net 4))
 (segment (start 186.86 92.67) (end 186.86 92.58) (width 0.25) (layer "F.Cu") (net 4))
 (segment (start 184.690989 94.839011) (end 186.1 93.43) (width 0.25) (layer "F.Cu") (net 4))
 (segment (start 183.465443 94.534557) (end 183.769897 94.839011) (width 0.25) (layer "F.Cu") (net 4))
 (segment (start 182.88 94.28904) (end 183.219926 94.28904) (width 0.25) (layer "F.Cu") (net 4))
 (segment (start 160.46 91.635) (end 163.11404 94.28904) (width 0.25) (layer "F.Cu") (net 4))
 (segment (start 186.1 93.43) (end 186.86 92.67) (width 0.25) (layer "F.Cu") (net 4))
 (segment (start 183.769897 94.839011) (end 184.690989 94.839011) (width 0.25) (layer "F.Cu") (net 4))
 (segment (start 164.55 94.28904) (end 182.88 94.28904) (width 0.25) (layer "F.Cu") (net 4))
 (via (at 186.86 92.58) (size 0.8) (drill 0.4) (layers "F.Cu" "B.Cu") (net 4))
 (segment (start 188.44 91) (end 189.76 91) (width 0.25) (layer "B.Cu") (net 4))
 (segment (start 186.86 92.58) (end 188.44 91) (width 0.25) (layer "B.Cu") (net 4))
 (segment (start 158.365489 91.189511) (end 159.19 90.365) (width 0.25) (layer "F.Cu") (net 9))
 (segment (start 189.51 95) (end 189.221469 95.288531) (width 0.25) (layer "F.Cu") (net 9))
 (segment (start 189.221469 95.288531) (end 183.583699 95.288531) (width 0.25) (layer "F.Cu") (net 9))
 (segment (start 158.365489 92.515489) (end 158.365489 91.189511) (width 0.25) (layer "F.Cu") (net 9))
 (segment (start 183.583699 95.288531) (end 183.033728 94.73856) (width 0.25) (layer "F.Cu") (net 9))
 (segment (start 183.033728 94.73856) (end 160.58856 94.73856) (width 0.25) (layer "F.Cu") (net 9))
 (segment (start 160.58856 94.73856) (end 158.365489 92.515489) (width 0.25) (layer "F.Cu") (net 9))
 (segment (start 183.59452 87.93548) (end 184.29 87.24) (width 0.25) (layer "F.Cu") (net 8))
 (segment (start 171.677027 88.62048) (end 172.362027 87.93548) (width 0.25) (layer "F.Cu") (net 8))
 (segment (start 158.074051 90.314913) (end 158.868964 89.52) (width 0.25) (layer "F.Cu") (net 8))
 (segment (start 158.074051 90.456351) (end 158.074051 90.314913) (width 0.25) (layer "F.Cu") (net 8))
 (segment (start 158.868964 89.52) (end 160.64 89.52) (width 0.25) (layer "F.Cu") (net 8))
 (segment (start 161.53952 88.62048) (end 171.677027 88.62048) (width 0.25) (layer "F.Cu") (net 8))
 (segment (start 172.362027 87.93548) (end 183.59452 87.93548) (width 0.25) (layer "F.Cu") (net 8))
 (segment (start 160.64 89.52) (end 161.53952 88.62048) (width 0.25) (layer "F.Cu") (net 8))
 (via (at 158.074051 90.456351) (size 0.8) (drill 0.4) (layers "F.Cu" "B.Cu") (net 8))
 (via (at 184.29 87.24) (size 0.8) (drill 0.4) (layers "F.Cu" "B.Cu") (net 8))
 (segment (start 184.29 87.24) (end 189.22 87.24) (width 0.25) (layer "B.Cu") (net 8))
 (segment (start 189.22 87.24) (end 189.46 87) (width 0.25) (layer "B.Cu") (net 8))
 (segment (start 159.19 91.635) (end 159.19 91.5723) (width 0.25) (layer "B.Cu") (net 8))
 (segment (start 159.19 91.5723) (end 158.074051 90.456351) (width 0.25) (layer "B.Cu") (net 8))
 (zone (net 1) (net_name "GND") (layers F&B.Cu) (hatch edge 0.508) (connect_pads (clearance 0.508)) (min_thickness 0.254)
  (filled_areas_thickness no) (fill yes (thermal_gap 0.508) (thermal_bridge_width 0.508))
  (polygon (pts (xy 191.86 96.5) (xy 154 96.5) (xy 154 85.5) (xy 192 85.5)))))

